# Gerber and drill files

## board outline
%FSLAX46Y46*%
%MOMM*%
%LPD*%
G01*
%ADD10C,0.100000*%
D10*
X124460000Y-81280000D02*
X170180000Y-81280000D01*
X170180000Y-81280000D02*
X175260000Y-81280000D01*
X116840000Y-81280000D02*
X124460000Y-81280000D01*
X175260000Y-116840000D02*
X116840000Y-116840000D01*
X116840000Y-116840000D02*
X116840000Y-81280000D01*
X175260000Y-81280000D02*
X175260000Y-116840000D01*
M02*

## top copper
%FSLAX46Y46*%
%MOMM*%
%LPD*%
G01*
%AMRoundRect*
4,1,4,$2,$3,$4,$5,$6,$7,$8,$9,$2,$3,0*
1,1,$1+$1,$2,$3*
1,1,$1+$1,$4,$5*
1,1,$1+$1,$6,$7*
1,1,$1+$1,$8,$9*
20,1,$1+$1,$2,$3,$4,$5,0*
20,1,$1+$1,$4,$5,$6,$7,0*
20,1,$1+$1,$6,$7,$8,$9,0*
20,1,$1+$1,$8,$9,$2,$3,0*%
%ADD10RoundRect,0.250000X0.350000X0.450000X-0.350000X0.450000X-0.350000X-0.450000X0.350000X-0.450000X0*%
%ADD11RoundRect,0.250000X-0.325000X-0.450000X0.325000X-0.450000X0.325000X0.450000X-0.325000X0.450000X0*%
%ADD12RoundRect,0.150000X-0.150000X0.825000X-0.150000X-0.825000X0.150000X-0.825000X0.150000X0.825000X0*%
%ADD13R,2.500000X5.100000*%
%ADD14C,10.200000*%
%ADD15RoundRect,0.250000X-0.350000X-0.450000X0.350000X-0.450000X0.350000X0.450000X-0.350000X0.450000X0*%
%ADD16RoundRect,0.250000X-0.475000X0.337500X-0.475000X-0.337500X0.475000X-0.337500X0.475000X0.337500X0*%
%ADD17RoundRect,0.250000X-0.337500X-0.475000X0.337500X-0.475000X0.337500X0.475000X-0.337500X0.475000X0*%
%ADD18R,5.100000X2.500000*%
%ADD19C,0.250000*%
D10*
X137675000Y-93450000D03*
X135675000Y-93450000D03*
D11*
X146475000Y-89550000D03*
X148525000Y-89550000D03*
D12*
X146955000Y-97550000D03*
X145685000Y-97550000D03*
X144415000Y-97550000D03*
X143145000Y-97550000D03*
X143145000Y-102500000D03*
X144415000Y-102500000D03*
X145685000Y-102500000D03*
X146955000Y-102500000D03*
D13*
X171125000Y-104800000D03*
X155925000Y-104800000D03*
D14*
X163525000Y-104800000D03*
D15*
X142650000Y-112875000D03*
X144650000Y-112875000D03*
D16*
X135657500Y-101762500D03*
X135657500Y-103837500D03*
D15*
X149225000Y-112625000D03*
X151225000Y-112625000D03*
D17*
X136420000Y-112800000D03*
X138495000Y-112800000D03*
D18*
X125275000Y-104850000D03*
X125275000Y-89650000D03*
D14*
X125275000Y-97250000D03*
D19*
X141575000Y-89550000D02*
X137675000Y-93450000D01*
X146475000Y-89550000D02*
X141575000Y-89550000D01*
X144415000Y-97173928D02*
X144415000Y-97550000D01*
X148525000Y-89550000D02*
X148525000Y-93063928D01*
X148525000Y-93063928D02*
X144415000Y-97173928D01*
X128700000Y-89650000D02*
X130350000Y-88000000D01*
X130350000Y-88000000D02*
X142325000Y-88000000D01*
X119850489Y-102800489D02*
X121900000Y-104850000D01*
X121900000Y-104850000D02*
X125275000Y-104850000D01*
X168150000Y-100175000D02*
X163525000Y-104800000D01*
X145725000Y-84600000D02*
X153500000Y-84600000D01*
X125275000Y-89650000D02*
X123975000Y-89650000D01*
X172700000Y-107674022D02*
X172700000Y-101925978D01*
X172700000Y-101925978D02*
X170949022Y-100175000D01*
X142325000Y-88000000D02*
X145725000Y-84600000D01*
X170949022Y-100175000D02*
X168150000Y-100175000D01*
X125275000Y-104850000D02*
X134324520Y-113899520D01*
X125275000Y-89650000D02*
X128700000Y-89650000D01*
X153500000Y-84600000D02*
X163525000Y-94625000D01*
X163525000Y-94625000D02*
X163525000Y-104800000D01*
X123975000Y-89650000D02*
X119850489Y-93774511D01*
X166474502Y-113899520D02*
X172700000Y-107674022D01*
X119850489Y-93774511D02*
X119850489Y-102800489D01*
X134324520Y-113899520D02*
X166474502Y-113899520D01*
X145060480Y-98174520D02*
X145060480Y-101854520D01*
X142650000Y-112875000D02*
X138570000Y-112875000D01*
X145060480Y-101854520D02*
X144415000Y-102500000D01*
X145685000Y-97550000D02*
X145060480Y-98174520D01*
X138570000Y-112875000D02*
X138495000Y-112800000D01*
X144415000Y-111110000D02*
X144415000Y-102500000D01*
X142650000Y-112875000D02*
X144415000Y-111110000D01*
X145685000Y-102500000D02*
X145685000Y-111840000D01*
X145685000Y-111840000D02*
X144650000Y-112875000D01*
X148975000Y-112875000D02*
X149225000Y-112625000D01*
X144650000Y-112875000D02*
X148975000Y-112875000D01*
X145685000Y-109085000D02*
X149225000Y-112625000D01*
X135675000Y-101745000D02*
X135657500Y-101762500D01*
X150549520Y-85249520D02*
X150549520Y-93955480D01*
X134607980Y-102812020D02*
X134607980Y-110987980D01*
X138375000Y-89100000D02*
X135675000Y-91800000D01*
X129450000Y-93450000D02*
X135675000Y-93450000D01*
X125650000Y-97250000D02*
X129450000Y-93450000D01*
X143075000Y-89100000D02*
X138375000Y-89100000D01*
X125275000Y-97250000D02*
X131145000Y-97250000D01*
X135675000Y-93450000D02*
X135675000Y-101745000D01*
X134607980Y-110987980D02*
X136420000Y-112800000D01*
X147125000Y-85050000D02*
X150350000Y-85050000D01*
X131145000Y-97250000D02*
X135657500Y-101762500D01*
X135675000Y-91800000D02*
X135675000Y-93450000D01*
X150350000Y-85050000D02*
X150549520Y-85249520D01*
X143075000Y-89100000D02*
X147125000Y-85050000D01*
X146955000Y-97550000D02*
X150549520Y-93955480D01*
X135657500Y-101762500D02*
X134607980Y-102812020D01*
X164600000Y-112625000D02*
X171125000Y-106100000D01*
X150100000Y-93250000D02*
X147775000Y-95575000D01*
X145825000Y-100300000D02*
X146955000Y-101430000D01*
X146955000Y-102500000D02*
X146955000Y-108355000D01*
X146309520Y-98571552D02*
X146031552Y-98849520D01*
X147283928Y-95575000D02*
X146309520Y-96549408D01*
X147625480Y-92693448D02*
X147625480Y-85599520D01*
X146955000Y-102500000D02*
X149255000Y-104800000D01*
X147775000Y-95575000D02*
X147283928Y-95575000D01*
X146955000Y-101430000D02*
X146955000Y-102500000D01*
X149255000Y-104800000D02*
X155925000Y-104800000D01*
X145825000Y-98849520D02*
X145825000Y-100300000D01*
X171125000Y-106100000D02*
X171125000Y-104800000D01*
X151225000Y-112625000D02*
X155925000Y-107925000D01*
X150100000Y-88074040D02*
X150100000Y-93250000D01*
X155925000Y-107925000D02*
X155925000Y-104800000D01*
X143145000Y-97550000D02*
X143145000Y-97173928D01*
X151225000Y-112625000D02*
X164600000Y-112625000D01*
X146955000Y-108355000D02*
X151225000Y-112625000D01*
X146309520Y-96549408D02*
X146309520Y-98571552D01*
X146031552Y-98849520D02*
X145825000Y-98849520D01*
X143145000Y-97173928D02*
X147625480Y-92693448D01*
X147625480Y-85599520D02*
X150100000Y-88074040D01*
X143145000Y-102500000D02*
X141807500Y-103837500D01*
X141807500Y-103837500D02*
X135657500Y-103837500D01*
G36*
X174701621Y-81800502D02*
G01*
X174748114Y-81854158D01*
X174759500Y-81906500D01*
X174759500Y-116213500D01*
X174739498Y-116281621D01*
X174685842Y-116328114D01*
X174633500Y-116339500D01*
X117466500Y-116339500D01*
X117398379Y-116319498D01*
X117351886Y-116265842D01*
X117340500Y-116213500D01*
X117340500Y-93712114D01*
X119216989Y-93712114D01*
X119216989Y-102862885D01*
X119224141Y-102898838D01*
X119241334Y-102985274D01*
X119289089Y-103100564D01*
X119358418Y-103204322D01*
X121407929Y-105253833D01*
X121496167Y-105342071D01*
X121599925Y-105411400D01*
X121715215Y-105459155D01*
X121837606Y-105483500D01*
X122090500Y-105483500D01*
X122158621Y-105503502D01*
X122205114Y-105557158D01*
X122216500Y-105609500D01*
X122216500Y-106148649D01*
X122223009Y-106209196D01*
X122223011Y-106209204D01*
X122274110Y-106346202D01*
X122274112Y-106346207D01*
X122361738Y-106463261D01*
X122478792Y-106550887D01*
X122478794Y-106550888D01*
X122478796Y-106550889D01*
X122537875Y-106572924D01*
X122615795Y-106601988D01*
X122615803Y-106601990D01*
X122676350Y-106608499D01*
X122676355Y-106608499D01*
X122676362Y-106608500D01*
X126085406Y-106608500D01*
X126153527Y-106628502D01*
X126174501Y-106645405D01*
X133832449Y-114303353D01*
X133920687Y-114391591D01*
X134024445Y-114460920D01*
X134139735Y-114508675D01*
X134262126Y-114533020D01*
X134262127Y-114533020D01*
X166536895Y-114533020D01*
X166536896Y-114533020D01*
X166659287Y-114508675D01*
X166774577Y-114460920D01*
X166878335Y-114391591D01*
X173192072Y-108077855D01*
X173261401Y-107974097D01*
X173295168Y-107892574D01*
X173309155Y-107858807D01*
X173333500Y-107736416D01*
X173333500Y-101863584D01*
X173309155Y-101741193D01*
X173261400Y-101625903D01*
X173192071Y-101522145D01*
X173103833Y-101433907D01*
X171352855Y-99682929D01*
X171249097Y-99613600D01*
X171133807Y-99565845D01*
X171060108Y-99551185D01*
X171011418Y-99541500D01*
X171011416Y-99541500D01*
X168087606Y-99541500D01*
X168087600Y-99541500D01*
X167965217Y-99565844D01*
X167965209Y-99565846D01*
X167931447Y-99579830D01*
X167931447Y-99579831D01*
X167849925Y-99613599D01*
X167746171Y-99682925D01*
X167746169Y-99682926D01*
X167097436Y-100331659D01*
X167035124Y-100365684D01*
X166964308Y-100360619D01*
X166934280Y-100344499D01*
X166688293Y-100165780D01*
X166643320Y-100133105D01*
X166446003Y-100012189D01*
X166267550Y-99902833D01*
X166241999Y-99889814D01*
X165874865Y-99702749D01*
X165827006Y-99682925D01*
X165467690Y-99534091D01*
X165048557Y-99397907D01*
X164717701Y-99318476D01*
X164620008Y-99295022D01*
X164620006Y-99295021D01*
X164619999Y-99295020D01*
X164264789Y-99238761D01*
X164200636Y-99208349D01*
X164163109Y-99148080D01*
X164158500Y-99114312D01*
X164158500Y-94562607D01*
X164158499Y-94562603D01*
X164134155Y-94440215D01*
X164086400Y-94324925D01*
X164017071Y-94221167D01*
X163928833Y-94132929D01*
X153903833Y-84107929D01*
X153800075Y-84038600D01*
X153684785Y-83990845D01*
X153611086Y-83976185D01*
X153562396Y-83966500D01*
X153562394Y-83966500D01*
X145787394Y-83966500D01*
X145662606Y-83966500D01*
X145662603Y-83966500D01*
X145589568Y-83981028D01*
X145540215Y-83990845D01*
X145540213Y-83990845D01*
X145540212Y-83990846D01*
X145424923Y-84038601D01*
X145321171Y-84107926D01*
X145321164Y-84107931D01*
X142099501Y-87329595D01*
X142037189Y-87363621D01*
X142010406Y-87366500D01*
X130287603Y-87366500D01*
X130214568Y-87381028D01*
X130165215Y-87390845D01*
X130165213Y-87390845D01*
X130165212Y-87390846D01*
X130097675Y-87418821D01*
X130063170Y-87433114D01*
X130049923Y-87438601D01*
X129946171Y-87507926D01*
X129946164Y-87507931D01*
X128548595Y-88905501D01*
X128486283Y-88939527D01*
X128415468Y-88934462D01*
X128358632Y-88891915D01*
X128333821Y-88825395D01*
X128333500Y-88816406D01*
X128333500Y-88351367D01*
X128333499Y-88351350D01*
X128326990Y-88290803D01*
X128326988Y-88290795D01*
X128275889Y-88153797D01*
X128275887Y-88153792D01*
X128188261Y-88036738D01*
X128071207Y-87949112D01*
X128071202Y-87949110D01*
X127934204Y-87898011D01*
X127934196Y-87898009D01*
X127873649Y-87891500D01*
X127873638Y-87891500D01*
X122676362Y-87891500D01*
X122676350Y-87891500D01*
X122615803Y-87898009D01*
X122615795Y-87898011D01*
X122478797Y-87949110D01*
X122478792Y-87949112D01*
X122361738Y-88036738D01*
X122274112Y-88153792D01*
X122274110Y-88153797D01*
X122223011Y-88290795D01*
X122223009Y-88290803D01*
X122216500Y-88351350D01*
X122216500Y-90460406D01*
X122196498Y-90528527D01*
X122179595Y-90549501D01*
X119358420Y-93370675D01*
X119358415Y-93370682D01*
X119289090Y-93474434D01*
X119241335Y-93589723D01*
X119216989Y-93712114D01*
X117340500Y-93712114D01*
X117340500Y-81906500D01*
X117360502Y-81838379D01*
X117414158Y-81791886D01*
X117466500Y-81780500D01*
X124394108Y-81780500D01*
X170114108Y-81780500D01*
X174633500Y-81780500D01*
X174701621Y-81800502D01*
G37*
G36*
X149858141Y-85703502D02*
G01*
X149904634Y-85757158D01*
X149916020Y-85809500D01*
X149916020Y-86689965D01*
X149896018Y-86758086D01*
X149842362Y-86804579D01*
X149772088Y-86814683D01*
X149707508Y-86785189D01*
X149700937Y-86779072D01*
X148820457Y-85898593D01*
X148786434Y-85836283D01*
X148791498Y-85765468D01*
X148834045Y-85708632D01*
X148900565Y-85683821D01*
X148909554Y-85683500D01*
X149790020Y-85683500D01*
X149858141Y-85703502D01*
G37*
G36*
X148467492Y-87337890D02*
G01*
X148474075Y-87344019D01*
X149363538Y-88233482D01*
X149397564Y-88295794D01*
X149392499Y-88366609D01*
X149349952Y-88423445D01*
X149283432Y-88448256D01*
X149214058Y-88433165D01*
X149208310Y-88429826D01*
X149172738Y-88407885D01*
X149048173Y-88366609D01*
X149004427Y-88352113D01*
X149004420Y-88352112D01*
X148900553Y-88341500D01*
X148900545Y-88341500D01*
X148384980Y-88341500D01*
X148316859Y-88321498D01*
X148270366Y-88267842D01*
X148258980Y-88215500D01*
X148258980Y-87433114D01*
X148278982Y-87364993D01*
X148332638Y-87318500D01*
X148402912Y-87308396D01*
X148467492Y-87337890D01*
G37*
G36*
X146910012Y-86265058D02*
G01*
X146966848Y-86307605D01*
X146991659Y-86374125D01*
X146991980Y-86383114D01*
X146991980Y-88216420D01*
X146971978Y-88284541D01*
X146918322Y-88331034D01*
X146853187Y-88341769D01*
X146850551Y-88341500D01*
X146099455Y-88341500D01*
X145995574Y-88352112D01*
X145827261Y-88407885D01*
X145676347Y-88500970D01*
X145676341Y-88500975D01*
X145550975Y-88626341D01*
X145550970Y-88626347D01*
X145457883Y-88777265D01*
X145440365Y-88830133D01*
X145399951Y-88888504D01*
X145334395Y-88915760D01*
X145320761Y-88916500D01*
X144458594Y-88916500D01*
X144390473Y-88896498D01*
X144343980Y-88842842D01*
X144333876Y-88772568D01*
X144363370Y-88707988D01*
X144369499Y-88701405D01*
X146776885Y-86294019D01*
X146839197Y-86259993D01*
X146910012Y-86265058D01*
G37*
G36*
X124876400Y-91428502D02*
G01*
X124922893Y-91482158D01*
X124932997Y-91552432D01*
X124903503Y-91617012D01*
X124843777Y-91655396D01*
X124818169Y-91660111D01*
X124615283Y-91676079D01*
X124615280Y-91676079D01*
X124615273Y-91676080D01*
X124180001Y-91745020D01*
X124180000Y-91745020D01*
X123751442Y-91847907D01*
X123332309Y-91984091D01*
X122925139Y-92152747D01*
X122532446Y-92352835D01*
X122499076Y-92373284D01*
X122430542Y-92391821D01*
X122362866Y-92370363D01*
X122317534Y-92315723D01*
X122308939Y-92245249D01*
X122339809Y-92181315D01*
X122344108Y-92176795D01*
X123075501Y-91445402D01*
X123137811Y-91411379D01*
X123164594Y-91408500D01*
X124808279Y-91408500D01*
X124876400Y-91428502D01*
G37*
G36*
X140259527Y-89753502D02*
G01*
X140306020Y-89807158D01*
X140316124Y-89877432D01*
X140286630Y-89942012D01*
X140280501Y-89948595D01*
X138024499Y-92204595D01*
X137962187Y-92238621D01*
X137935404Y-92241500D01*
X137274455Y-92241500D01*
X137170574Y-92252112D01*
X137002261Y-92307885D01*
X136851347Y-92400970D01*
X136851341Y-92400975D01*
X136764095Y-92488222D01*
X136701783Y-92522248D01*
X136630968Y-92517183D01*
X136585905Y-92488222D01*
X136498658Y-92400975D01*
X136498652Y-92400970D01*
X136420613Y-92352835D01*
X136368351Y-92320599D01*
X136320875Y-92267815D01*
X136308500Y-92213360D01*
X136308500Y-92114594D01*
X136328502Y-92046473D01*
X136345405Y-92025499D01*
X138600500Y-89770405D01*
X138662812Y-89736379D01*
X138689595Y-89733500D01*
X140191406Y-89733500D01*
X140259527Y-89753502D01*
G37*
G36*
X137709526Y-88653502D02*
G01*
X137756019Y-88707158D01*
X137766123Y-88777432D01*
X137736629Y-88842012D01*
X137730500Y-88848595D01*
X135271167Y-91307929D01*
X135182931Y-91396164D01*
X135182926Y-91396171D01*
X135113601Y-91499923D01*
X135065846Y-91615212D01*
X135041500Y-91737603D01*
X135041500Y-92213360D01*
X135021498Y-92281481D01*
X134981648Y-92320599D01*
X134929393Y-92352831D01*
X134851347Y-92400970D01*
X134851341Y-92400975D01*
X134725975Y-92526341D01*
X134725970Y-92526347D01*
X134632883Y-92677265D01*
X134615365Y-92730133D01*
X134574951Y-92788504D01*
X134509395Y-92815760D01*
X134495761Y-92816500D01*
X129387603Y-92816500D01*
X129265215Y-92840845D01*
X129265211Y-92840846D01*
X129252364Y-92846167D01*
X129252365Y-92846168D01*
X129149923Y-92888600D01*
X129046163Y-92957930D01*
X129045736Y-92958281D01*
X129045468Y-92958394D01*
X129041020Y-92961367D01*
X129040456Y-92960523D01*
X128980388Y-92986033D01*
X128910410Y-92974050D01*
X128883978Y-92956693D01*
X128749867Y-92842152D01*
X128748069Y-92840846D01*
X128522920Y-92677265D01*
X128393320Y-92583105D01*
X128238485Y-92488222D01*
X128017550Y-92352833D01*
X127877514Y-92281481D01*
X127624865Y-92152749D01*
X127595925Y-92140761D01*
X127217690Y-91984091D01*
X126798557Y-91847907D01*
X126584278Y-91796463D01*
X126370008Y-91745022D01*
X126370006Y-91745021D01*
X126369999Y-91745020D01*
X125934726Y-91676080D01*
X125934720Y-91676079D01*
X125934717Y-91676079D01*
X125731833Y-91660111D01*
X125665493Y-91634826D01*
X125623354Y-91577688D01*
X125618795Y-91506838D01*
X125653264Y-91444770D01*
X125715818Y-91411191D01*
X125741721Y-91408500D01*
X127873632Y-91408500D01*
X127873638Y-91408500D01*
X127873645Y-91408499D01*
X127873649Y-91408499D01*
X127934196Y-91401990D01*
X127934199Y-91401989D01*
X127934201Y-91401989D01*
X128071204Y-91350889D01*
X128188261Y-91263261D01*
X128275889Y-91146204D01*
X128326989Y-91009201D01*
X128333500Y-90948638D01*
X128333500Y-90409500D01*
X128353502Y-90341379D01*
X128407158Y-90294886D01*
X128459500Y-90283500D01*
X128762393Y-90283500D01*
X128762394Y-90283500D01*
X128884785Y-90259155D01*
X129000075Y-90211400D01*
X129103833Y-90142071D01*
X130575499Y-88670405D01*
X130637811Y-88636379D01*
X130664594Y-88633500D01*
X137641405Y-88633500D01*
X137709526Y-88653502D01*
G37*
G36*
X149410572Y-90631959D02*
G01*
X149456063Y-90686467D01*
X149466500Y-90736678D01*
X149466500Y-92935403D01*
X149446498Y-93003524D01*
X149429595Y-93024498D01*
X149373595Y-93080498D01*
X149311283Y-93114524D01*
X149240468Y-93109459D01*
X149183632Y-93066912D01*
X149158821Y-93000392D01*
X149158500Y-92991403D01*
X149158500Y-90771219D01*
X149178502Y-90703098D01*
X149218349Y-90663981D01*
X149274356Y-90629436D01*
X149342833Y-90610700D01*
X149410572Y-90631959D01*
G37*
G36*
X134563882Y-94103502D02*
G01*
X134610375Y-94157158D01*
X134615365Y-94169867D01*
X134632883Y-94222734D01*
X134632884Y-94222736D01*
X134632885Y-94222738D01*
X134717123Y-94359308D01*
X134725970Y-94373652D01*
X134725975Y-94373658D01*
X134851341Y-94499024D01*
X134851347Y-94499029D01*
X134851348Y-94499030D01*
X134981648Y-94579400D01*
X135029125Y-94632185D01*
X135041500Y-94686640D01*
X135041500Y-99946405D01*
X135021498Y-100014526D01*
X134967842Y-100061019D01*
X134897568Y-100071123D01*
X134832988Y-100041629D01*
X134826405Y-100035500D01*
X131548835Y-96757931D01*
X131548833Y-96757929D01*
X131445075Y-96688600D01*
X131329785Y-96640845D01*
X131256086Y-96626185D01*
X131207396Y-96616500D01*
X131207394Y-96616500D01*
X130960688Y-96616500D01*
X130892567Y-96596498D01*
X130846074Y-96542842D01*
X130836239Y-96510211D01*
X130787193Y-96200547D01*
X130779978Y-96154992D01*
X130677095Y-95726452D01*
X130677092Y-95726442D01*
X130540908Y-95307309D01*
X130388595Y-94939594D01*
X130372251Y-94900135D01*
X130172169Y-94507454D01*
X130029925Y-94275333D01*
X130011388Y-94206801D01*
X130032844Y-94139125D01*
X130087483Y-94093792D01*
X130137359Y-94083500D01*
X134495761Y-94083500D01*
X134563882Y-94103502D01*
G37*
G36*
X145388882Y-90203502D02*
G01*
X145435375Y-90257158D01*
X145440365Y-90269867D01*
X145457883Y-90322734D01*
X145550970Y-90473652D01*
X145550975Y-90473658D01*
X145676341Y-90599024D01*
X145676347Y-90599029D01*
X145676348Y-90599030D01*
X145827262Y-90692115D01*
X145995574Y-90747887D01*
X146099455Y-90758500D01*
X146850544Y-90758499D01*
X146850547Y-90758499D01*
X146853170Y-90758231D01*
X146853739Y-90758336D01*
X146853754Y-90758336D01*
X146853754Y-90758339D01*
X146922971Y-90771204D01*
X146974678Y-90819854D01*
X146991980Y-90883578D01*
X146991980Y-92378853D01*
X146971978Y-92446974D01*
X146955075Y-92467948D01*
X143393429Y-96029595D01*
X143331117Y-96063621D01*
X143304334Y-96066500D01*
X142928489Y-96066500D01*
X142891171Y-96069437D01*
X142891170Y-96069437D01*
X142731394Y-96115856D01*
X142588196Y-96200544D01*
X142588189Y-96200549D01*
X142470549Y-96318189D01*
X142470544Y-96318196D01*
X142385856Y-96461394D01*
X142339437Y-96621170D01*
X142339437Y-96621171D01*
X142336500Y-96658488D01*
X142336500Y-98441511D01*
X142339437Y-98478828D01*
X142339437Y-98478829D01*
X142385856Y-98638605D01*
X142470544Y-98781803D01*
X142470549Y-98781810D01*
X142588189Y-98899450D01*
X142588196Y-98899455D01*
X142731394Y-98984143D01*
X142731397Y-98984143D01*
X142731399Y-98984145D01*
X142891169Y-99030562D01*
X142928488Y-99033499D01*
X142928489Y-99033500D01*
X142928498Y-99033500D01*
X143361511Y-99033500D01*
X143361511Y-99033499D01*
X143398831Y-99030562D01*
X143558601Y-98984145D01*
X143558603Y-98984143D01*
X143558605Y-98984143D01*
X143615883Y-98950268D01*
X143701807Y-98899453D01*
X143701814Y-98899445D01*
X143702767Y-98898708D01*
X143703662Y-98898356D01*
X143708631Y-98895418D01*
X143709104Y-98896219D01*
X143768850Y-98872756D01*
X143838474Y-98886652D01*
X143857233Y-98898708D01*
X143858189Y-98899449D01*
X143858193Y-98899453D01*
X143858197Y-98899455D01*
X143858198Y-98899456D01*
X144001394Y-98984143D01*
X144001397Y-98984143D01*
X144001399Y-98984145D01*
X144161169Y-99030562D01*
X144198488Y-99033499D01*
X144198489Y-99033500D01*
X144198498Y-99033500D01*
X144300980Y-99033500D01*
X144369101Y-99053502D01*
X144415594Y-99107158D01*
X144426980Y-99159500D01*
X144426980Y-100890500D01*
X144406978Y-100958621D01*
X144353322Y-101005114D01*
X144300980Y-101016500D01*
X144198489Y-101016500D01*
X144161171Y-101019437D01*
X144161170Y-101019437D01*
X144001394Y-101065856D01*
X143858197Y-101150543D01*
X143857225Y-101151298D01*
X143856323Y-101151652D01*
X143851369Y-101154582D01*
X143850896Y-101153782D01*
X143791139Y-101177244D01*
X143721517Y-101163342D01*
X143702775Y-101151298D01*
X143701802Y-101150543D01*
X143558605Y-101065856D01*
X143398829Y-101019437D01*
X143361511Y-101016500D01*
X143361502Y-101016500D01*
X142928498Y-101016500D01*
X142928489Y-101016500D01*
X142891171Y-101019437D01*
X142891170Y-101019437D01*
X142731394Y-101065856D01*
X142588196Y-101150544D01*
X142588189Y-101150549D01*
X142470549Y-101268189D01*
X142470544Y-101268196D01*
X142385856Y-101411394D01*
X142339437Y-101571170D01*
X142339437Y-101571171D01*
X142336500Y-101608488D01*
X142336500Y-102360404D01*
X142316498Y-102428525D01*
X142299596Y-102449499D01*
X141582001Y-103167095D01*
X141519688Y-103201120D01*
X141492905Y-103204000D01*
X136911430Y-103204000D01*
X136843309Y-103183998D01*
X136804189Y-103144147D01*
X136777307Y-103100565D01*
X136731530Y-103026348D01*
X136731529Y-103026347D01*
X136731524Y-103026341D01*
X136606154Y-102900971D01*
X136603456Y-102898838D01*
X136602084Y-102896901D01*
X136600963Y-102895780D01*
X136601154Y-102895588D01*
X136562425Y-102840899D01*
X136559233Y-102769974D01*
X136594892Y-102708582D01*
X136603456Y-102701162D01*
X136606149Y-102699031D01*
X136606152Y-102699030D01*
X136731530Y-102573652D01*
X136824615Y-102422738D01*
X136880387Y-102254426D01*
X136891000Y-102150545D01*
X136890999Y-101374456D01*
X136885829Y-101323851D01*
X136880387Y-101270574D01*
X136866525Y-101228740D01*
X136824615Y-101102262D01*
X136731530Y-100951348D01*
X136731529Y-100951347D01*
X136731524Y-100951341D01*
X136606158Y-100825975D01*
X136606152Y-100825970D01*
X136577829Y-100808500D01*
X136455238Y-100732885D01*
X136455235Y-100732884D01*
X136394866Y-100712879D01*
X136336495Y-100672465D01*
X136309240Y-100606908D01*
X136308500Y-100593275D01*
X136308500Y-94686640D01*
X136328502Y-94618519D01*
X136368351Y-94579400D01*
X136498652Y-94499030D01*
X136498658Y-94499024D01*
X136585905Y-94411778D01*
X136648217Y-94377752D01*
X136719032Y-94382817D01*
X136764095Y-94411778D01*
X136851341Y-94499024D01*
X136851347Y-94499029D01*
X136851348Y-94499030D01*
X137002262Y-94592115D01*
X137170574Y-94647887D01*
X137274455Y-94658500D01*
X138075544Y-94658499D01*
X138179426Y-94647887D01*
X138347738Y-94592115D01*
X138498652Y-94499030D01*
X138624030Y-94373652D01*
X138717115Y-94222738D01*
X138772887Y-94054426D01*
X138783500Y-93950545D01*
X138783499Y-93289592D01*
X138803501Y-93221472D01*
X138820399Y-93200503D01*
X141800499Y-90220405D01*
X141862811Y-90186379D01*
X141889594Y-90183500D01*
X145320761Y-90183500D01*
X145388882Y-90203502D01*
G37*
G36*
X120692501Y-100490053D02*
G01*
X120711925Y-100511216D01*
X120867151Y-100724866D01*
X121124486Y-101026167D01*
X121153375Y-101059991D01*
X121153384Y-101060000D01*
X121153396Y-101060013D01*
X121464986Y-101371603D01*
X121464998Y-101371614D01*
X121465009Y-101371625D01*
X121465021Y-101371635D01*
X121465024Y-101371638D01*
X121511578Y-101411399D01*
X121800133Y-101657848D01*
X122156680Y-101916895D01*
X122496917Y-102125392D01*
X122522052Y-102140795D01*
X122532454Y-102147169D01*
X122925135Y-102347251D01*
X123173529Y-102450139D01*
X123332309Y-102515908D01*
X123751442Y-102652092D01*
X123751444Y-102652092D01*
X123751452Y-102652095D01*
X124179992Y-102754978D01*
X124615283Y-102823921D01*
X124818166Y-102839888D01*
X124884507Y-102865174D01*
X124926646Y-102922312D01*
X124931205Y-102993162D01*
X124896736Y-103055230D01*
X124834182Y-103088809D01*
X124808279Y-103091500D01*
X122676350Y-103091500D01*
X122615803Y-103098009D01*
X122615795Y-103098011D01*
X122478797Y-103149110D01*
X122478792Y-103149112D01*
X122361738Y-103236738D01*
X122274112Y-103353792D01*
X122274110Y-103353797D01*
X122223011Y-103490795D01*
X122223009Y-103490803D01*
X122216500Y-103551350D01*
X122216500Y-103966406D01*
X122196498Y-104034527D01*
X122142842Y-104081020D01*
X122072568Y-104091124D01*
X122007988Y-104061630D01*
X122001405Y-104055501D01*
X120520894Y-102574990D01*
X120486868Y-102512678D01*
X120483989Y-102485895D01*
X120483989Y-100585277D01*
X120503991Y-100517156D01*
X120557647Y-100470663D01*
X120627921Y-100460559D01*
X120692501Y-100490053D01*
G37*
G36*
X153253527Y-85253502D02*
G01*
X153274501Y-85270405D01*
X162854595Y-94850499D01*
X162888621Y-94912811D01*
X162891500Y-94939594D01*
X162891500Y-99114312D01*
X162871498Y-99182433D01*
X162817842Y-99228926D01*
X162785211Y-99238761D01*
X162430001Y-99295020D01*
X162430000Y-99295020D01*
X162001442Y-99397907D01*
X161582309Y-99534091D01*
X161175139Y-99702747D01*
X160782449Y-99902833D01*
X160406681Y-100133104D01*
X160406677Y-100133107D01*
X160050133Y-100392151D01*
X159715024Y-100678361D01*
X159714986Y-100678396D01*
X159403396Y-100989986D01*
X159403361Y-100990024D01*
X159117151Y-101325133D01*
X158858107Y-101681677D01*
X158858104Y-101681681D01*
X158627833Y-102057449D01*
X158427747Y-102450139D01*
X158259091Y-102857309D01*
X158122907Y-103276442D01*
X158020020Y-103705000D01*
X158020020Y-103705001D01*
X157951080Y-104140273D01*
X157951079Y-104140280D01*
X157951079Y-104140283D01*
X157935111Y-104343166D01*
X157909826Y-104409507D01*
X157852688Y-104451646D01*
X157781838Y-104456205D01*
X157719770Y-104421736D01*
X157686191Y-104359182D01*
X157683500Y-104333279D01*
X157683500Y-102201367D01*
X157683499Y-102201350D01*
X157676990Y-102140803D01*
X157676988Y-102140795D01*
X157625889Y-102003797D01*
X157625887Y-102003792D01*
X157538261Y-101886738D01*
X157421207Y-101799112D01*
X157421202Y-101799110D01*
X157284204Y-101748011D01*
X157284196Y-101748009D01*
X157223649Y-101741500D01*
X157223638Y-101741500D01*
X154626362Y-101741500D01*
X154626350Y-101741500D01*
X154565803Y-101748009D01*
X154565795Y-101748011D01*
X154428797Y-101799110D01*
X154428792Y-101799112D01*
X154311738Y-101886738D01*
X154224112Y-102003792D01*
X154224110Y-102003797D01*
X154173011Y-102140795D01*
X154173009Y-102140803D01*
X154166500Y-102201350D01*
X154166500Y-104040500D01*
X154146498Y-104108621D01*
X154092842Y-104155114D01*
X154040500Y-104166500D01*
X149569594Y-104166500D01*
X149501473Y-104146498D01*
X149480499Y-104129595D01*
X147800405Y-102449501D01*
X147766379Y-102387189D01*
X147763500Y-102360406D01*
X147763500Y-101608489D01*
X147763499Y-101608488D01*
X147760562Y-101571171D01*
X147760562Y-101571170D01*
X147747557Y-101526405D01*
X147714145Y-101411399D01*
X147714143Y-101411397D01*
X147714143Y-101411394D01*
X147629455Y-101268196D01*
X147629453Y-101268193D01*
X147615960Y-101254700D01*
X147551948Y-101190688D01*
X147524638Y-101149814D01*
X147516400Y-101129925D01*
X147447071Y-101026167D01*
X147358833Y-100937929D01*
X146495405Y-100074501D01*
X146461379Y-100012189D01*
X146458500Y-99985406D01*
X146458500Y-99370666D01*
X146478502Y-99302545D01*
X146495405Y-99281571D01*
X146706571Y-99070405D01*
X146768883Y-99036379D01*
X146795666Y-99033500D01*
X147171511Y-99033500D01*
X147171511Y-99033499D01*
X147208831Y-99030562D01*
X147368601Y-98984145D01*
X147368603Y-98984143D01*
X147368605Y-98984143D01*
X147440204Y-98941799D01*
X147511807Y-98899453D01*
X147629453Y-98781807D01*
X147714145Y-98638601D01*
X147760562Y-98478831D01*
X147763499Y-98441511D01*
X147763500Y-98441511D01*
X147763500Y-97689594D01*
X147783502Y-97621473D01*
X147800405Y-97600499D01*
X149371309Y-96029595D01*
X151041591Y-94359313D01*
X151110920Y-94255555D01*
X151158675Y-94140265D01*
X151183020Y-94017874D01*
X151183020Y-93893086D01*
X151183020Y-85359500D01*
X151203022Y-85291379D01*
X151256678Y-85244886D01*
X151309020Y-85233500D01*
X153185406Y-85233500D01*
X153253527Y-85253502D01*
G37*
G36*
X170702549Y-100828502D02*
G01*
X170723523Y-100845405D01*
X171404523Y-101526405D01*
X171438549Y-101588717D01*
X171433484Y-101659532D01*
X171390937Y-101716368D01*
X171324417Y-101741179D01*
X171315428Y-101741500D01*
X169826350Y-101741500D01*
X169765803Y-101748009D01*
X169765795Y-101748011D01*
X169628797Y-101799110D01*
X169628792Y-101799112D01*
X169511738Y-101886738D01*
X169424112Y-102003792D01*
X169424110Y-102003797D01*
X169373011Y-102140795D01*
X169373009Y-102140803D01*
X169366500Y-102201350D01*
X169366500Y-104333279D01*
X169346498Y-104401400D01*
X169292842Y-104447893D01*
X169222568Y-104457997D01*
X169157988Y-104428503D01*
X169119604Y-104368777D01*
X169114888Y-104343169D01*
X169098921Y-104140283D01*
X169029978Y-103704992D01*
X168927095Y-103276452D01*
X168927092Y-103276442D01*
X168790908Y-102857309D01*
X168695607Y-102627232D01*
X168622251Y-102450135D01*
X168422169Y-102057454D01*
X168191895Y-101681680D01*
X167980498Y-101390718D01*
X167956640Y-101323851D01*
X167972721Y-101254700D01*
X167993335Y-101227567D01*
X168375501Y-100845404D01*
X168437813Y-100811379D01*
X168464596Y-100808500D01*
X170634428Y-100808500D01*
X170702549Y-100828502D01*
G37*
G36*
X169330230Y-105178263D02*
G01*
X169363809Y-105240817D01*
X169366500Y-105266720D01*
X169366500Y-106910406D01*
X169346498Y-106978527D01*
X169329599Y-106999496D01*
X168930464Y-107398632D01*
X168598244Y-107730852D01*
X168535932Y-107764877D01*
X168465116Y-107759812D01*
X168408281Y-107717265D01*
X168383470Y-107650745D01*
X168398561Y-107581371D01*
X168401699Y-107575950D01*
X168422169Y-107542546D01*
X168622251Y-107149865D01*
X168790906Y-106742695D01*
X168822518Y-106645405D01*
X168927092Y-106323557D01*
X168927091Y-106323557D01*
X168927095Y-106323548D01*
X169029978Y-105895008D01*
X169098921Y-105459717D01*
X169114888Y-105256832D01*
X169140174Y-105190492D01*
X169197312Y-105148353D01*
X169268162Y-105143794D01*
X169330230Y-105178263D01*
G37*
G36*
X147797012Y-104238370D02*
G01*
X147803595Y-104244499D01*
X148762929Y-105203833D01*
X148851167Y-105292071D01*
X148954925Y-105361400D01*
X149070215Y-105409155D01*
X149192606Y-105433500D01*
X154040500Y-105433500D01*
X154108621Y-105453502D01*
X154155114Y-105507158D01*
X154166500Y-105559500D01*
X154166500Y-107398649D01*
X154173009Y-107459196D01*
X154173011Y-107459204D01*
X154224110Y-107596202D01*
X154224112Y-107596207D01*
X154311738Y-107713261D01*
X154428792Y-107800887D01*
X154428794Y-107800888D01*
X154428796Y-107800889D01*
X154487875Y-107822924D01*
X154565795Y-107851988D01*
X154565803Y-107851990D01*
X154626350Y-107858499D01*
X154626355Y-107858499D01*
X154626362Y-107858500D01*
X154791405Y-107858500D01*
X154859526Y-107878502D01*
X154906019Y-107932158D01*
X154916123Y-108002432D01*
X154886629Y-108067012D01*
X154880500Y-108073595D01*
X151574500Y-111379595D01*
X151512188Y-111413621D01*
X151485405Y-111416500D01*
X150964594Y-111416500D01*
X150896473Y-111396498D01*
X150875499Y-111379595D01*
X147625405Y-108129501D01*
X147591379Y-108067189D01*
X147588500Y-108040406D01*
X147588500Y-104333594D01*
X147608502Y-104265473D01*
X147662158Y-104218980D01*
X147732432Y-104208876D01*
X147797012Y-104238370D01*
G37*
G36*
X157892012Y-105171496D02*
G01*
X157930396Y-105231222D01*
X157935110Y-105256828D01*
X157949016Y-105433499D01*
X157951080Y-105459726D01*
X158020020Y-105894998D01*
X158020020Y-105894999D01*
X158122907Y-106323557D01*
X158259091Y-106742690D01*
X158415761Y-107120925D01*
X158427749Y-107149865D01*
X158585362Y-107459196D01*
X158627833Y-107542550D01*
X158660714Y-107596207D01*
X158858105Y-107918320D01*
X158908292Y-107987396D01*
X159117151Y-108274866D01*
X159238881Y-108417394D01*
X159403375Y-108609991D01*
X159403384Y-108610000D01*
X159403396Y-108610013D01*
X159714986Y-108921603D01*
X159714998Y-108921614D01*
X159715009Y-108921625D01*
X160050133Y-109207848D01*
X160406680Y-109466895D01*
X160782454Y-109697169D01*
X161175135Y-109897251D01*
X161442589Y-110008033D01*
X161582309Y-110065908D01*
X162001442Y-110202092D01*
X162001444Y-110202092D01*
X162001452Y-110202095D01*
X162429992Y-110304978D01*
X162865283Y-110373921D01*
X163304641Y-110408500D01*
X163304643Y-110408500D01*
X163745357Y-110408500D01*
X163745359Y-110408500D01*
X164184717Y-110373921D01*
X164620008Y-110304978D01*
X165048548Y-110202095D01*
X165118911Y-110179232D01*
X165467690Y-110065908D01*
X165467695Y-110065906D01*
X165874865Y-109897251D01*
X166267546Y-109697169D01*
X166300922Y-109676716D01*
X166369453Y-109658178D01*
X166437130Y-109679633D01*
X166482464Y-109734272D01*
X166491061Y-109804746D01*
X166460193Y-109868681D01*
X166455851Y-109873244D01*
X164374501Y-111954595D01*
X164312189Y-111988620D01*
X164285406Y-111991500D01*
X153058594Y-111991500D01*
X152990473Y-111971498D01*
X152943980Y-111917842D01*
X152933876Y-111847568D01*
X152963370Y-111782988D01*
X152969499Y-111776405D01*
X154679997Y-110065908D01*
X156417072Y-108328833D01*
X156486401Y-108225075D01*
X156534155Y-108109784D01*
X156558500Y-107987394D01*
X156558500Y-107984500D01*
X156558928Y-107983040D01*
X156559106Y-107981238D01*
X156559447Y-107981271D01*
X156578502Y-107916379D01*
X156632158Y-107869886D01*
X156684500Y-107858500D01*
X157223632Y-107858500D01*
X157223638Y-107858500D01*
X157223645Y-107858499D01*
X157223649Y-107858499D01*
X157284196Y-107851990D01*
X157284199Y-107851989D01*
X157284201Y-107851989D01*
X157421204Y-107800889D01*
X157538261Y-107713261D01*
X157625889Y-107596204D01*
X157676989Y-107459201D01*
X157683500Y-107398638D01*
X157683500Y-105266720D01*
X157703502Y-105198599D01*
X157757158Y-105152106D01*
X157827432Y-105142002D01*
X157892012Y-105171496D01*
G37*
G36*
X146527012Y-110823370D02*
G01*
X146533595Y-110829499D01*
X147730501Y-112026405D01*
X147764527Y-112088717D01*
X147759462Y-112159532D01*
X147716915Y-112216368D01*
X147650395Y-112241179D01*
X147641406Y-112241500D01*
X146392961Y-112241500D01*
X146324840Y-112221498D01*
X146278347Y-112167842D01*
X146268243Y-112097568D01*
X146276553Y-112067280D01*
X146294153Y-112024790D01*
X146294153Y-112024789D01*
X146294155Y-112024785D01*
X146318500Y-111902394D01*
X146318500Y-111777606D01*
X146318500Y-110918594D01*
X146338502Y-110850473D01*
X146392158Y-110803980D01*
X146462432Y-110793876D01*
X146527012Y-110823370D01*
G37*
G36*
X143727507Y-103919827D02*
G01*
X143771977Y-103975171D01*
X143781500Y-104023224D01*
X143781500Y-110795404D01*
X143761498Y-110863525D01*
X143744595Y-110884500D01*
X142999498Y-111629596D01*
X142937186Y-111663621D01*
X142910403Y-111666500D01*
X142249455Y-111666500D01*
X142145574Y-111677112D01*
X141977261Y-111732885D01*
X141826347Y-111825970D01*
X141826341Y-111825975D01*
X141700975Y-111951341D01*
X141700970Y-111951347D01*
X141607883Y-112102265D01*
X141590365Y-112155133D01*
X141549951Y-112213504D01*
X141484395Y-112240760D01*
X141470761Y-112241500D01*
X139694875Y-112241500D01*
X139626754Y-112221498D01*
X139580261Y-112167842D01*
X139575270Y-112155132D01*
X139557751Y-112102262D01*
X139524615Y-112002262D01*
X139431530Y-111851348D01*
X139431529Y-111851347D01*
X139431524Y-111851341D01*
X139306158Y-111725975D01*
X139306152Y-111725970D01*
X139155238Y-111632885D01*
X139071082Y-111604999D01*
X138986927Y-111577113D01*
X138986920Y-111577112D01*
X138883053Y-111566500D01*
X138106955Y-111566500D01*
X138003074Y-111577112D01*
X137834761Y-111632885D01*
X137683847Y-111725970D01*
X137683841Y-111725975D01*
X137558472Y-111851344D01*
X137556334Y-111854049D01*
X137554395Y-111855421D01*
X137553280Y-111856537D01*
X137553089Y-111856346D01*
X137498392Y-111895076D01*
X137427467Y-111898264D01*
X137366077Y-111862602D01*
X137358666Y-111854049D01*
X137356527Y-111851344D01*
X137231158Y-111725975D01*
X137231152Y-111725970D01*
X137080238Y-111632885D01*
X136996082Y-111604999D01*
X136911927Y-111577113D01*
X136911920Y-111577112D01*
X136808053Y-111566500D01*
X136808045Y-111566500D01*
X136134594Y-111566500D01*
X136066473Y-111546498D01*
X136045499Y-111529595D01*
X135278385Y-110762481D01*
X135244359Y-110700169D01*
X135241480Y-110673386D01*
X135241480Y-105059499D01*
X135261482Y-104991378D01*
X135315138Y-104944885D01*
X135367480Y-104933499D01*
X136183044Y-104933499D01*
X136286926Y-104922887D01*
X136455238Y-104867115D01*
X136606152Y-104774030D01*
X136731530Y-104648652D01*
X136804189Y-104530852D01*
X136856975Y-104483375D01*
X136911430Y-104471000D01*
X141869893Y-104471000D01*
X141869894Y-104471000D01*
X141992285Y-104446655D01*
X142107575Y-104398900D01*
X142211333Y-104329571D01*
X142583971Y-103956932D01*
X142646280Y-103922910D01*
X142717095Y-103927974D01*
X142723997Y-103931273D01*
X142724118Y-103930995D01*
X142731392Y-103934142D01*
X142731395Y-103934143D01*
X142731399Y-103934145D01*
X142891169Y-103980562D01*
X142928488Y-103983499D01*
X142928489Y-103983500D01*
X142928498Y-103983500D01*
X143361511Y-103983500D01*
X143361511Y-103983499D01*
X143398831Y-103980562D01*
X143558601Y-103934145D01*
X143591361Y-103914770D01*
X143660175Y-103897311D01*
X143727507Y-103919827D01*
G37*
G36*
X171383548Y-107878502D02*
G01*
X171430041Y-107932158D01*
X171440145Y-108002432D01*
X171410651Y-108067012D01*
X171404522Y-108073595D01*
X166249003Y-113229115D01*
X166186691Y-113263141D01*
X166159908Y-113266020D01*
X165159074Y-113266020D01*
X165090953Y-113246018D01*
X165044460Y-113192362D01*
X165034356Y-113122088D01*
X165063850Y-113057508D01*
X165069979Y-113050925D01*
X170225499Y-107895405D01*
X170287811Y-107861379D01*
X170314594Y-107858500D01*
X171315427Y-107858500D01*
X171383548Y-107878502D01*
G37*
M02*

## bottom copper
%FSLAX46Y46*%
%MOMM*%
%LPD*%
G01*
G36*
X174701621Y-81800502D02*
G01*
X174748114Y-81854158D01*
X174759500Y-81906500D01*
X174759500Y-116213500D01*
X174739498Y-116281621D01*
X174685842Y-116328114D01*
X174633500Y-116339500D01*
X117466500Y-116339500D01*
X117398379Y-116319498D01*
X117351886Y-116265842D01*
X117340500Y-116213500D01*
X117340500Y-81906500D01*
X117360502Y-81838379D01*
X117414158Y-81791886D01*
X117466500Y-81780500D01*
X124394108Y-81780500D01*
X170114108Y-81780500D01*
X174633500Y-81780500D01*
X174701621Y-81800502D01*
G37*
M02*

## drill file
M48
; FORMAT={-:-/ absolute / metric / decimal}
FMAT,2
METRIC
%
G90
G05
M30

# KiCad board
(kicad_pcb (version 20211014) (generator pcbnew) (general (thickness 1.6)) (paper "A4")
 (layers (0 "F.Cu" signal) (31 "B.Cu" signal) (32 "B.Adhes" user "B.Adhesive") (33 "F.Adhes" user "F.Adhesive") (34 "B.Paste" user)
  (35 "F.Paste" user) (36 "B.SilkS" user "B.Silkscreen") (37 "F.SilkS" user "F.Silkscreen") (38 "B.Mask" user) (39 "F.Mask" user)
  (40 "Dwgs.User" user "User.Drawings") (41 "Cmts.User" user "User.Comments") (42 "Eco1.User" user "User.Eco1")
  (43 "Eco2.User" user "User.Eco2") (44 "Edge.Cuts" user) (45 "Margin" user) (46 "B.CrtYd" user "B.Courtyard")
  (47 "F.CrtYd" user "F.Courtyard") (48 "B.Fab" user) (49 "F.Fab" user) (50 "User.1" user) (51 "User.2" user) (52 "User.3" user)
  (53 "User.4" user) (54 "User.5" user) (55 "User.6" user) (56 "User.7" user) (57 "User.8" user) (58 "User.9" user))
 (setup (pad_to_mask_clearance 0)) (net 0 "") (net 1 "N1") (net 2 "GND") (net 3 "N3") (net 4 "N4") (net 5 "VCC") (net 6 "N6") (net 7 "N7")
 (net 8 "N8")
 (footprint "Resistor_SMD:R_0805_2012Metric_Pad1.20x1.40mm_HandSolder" (layer "F.Cu") (at 136.675 93.45 180)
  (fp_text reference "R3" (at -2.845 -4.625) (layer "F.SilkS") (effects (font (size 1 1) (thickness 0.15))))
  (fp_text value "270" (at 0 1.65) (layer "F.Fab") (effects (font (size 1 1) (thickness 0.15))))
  (pad "1" smd roundrect (at -1 0 180) (size 1.2 1.4) (layers "F.Cu" "F.Paste" "F.Mask") (roundrect_rratio 0.2083333333) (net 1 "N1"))
  (pad "2" smd roundrect (at 1 0 180) (size 1.2 1.4) (layers "F.Cu" "F.Paste" "F.Mask") (roundrect_rratio 0.2083333333) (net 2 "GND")))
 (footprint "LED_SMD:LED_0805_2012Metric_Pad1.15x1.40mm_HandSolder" (layer "F.Cu") (at 147.5 89.55)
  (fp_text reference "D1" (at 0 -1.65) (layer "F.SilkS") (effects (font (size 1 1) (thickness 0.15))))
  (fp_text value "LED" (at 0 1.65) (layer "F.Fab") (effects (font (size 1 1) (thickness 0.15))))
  (pad "1" smd roundrect (at -1.025 0) (size 1.15 1.4) (layers "F.Cu" "F.Paste" "F.Mask") (roundrect_rratio 0.2173913043) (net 1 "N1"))
  (pad "2" smd roundrect (at 1.025 0) (size 1.15 1.4) (layers "F.Cu" "F.Paste" "F.Mask") (roundrect_rratio 0.2173913043) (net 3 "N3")))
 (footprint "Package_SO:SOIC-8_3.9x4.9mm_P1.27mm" (layer "F.Cu") (at 145.05 100.025 -90)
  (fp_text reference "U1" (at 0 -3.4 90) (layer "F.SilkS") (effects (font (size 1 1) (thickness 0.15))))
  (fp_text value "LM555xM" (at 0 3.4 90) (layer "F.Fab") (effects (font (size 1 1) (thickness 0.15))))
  (pad "1" smd roundrect (at -2.475 -1.905 270) (size 1.95 0.6) (layers "F.Cu" "F.Paste" "F.Mask") (roundrect_rratio 0.25) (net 2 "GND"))
  (pad "2" smd roundrect (at -2.475 -0.635 270) (size 1.95 0.6) (layers "F.Cu" "F.Paste" "F.Mask") (roundrect_rratio 0.25) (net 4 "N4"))
  (pad "3" smd roundrect (at -2.475 0.635 270) (size 1.95 0.6) (layers "F.Cu" "F.Paste" "F.Mask") (roundrect_rratio 0.25) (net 3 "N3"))
  (pad "4" smd roundrect (at -2.475 1.905 270) (size 1.95 0.6) (layers "F.Cu" "F.Paste" "F.Mask") (roundrect_rratio 0.25) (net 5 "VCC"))
  (pad "5" smd roundrect (at 2.475 1.905 270) (size 1.95 0.6) (layers "F.Cu" "F.Paste" "F.Mask") (roundrect_rratio 0.25) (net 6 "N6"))
  (pad "6" smd roundrect (at 2.475 0.635 270) (size 1.95 0.6) (layers "F.Cu" "F.Paste" "F.Mask") (roundrect_rratio 0.25) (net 4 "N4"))
  (pad "7" smd roundrect (at 2.475 -0.635 270) (size 1.95 0.6) (layers "F.Cu" "F.Paste" "F.Mask") (roundrect_rratio 0.25) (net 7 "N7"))
  (pad "8" smd roundrect (at 2.475 -1.905 270) (size 1.95 0.6) (layers "F.Cu" "F.Paste" "F.Mask") (roundrect_rratio 0.25) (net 5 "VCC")))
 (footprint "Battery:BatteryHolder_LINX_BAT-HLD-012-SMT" (layer "F.Cu") (at 163.525 104.8 180)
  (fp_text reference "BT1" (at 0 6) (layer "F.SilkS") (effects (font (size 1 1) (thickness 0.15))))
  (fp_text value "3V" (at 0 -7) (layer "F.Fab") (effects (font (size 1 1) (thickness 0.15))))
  (pad "1" smd rect (at -7.6 0 180) (size 2.5 5.1) (layers "F.Cu" "F.Paste" "F.Mask") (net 5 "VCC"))
  (pad "1" smd rect (at 7.6 0 180) (size 2.5 5.1) (layers "F.Cu" "F.Paste" "F.Mask") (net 5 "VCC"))
  (pad "2" smd circle (at 0 0 180) (size 10.2 10.2) (layers "F.Cu" "F.Mask") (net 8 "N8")))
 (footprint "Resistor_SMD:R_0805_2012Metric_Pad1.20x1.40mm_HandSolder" (layer "F.Cu") (at 143.65 112.875)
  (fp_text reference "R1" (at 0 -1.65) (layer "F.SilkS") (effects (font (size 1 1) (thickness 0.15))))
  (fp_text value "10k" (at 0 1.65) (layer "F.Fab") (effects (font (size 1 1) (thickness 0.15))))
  (pad "1" smd roundrect (at -1 0) (size 1.2 1.4) (layers "F.Cu" "F.Paste" "F.Mask") (roundrect_rratio 0.2083333333) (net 4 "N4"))
  (pad "2" smd roundrect (at 1 0) (size 1.2 1.4) (layers "F.Cu" "F.Paste" "F.Mask") (roundrect_rratio 0.2083333333) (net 7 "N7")))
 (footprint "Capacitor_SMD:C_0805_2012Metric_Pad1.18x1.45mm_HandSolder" (layer "F.Cu") (at 135.6575 102.8 -90)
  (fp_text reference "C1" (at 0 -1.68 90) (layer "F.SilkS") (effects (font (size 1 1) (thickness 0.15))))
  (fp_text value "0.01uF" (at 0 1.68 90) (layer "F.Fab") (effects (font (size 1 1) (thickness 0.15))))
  (pad "1" smd roundrect (at -1.0375 0 270) (size 1.175 1.45) (layers "F.Cu" "F.Paste" "F.Mask") (roundrect_rratio 0.2127659574)
   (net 2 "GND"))
  (pad "2" smd roundrect (at 1.0375 0 270) (size 1.175 1.45) (layers "F.Cu" "F.Paste" "F.Mask") (roundrect_rratio 0.2127659574) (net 6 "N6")))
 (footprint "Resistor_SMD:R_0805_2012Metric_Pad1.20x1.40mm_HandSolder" (layer "F.Cu") (at 150.225 112.625)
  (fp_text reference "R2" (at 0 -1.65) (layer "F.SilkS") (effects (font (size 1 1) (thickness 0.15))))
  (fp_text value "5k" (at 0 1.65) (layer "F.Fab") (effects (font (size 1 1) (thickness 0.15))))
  (pad "1" smd roundrect (at -1 0) (size 1.2 1.4) (layers "F.Cu" "F.Paste" "F.Mask") (roundrect_rratio 0.2083333333) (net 7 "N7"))
  (pad "2" smd roundrect (at 1 0) (size 1.2 1.4) (layers "F.Cu" "F.Paste" "F.Mask") (roundrect_rratio 0.2083333333) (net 5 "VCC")))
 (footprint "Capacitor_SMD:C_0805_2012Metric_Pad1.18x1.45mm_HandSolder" (layer "F.Cu") (at 137.4575 112.8)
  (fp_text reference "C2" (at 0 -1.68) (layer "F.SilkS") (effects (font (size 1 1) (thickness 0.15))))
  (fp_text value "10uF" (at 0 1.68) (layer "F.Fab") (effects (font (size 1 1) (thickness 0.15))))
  (pad "1" smd roundrect (at -1.0375 0) (size 1.175 1.45) (layers "F.Cu" "F.Paste" "F.Mask") (roundrect_rratio 0.2127659574) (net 2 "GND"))
  (pad "2" smd roundrect (at 1.0375 0) (size 1.175 1.45) (layers "F.Cu" "F.Paste" "F.Mask") (roundrect_rratio 0.2127659574) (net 4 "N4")))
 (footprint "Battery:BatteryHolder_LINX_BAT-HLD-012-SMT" (layer "F.Cu") (at 125.275 97.25 -90)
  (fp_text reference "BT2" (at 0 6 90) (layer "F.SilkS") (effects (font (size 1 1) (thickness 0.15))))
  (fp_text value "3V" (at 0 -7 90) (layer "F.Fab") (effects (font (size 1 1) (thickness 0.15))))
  (pad "1" smd rect (at 7.6 0 270) (size 2.5 5.1) (layers "F.Cu" "F.Paste" "F.Mask") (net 8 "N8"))
  (pad "1" smd rect (at -7.6 0 270) (size 2.5 5.1) (layers "F.Cu" "F.Paste" "F.Mask") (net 8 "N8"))
  (pad "2" smd circle (at 0 0 270) (size 10.2 10.2) (layers "F.Cu" "F.Mask") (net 2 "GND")))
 (gr_line (start 124.46 81.28) (end 170.18 81.28) (layer "Edge.Cuts") (width 0.1))
 (gr_line (start 170.18 81.28) (end 175.26 81.28) (layer "Edge.Cuts") (width 0.1))
 (gr_line (start 116.84 81.28) (end 124.46 81.28) (layer "Edge.Cuts") (width 0.1))
 (gr_line (start 175.26 116.84) (end 116.84 116.84) (layer "Edge.Cuts") (width 0.1))
 (gr_line (start 116.84 116.84) (end 116.84 81.28) (layer "Edge.Cuts") (width 0.1))
 (gr_line (start 175.26 81.28) (end 175.26 116.84) (layer "Edge.Cuts") (width 0.1))
 (segment (start 141.575 89.55) (end 137.675 93.45) (width 0.25) (layer "F.Cu") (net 1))
 (segment (start 146.475 89.55) (end 141.575 89.55) (width 0.25) (layer "F.Cu") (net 1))
 (segment (start 144.415 97.173928) (end 144.415 97.55) (width 0.25) (layer "F.Cu") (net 3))
 (segment (start 148.525 89.55) (end 148.525 93.063928) (width 0.25) (layer "F.Cu") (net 3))
 (segment (start 148.525 93.063928) (end 144.415 97.173928) (width 0.25) (layer "F.Cu") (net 3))
 (segment (start 128.7 89.65) (end 130.35 88) (width 0.25) (layer "F.Cu") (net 8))
 (segment (start 130.35 88) (end 142.325 88) (width 0.25) (layer "F.Cu") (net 8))
 (segment (start 119.850489 102.800489) (end 121.9 104.85) (width 0.25) (layer "F.Cu") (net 8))
 (segment (start 121.9 104.85) (end 125.275 104.85) (width 0.25) (layer "F.Cu") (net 8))
 (segment (start 168.15 100.175) (end 163.525 104.8) (width 0.25) (layer "F.Cu") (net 8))
 (segment (start 145.725 84.6) (end 153.5 84.6) (width 0.25) (layer "F.Cu") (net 8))
 (segment (start 125.275 89.65) (end 123.975 89.65) (width 0.25) (layer "F.Cu") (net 8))
 (segment (start 172.7 107.674022) (end 172.7 101.925978) (width 0.25) (layer "F.Cu") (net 8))
 (segment (start 172.7 101.925978) (end 170.949022 100.175) (width 0.25) (layer "F.Cu") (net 8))
 (segment (start 142.325 88) (end 145.725 84.6) (width 0.25) (layer "F.Cu") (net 8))
 (segment (start 170.949022 100.175) (end 168.15 100.175) (width 0.25) (layer "F.Cu") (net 8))
 (segment (start 125.275 104.85) (end 134.32452 113.89952) (width 0.25) (layer "F.Cu") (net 8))
 (segment (start 125.275 89.65) (end 128.7 89.65) (width 0.25) (layer "F.Cu") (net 8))
 (segment (start 153.5 84.6) (end 163.525 94.625) (width 0.25) (layer "F.Cu") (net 8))
 (segment (start 163.525 94.625) (end 163.525 104.8) (width 0.25) (layer "F.Cu") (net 8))
 (segment (start 123.975 89.65) (end 119.850489 93.774511) (width 0.25) (layer "F.Cu") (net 8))
 (segment (start 166.474502 113.89952) (end 172.7 107.674022) (width 0.25) (layer "F.Cu") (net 8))
 (segment (start 119.850489 93.774511) (end 119.850489 102.800489) (width 0.25) (layer "F.Cu") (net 8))
 (segment (start 134.32452 113.89952) (end 166.474502 113.89952) (width 0.25) (layer "F.Cu") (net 8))
 (segment (start 145.06048 98.17452) (end 145.06048 101.85452) (width 0.25) (layer "F.Cu") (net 4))
 (segment (start 142.65 112.875) (end 138.57 112.875) (width 0.25) (layer "F.Cu") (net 4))
 (segment (start 145.06048 101.85452) (end 144.415 102.5) (width 0.25) (layer "F.Cu") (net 4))
 (segment (start 145.685 97.55) (end 145.06048 98.17452) (width 0.25) (layer "F.Cu") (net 4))
 (segment (start 138.57 112.875) (end 138.495 112.8) (width 0.25) (layer "F.Cu") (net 4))
 (segment (start 144.415 111.11) (end 144.415 102.5) (width 0.25) (layer "F.Cu") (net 4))
 (segment (start 142.65 112.875) (end 144.415 111.11) (width 0.25) (layer "F.Cu") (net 4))
 (segment (start 145.685 102.5) (end 145.685 111.84) (width 0.25) (layer "F.Cu") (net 7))
 (segment (start 145.685 111.84) (end 144.65 112.875) (width 0.25) (layer "F.Cu") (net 7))
 (segment (start 148.975 112.875) (end 149.225 112.625) (width 0.25) (layer "F.Cu") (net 7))
 (segment (start 144.65 112.875) (end 148.975 112.875) (width 0.25) (layer "F.Cu") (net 7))
 (segment (start 145.685 109.085) (end 149.225 112.625) (width 0.25) (layer "F.Cu") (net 7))
 (segment (start 135.675 101.745) (end 135.6575 101.7625) (width 0.25) (layer "F.Cu") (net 2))
 (segment (start 150.54952 85.24952) (end 150.54952 93.95548) (width 0.25) (layer "F.Cu") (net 2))
 (segment (start 134.60798 102.81202) (end 134.60798 110.98798) (width 0.25) (layer "F.Cu") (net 2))
 (segment (start 138.375 89.1) (end 135.675 91.8) (width 0.25) (layer "F.Cu") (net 2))
 (segment (start 129.45 93.45) (end 135.675 93.45) (width 0.25) (layer "F.Cu") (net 2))
 (segment (start 125.65 97.25) (end 129.45 93.45) (width 0.25) (layer "F.Cu") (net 2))
 (segment (start 143.075 89.1) (end 138.375 89.1) (width 0.25) (layer "F.Cu") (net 2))
 (segment (start 125.275 97.25) (end 131.145 97.25) (width 0.25) (layer "F.Cu") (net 2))
 (segment (start 135.675 93.45) (end 135.675 101.745) (width 0.25) (layer "F.Cu") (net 2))
 (segment (start 134.60798 110.98798) (end 136.42 112.8) (width 0.25) (layer "F.Cu") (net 2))
 (segment (start 147.125 85.05) (end 150.35 85.05) (width 0.25) (layer "F.Cu") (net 2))
 (segment (start 131.145 97.25) (end 135.6575 101.7625) (width 0.25) (layer "F.Cu") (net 2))
 (segment (start 135.675 91.8) (end 135.675 93.45) (width 0.25) (layer "F.Cu") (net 2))
 (segment (start 150.35 85.05) (end 150.54952 85.24952) (width 0.25) (layer "F.Cu") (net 2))
 (segment (start 143.075 89.1) (end 147.125 85.05) (width 0.25) (layer "F.Cu") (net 2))
 (segment (start 146.955 97.55) (end 150.54952 93.95548) (width 0.25) (layer "F.Cu") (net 2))
 (segment (start 135.6575 101.7625) (end 134.60798 102.81202) (width 0.25) (layer "F.Cu") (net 2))
 (segment (start 164.6 112.625) (end 171.125 106.1) (width 0.25) (layer "F.Cu") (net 5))
 (segment (start 150.1 93.25) (end 147.775 95.575) (width 0.25) (layer "F.Cu") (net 5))
 (segment (start 145.825 100.3) (end 146.955 101.43) (width 0.25) (layer "F.Cu") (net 5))
 (segment (start 146.955 102.5) (end 146.955 108.355) (width 0.25) (layer "F.Cu") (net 5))
 (segment (start 146.30952 98.571552) (end 146.031552 98.84952) (width 0.25) (layer "F.Cu") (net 5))
 (segment (start 147.283928 95.575) (end 146.30952 96.549408) (width 0.25) (layer "F.Cu") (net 5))
 (segment (start 147.62548 92.693448) (end 147.62548 85.59952) (width 0.25) (layer "F.Cu") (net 5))
 (segment (start 146.955 102.5) (end 149.255 104.8) (width 0.25) (layer "F.Cu") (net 5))
 (segment (start 147.775 95.575) (end 147.283928 95.575) (width 0.25) (layer "F.Cu") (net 5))
 (segment (start 146.955 101.43) (end 146.955 102.5) (width 0.25) (layer "F.Cu") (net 5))
 (segment (start 149.255 104.8) (end 155.925 104.8) (width 0.25) (layer "F.Cu") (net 5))
 (segment (start 145.825 98.84952) (end 145.825 100.3) (width 0.25) (layer "F.Cu") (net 5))
 (segment (start 171.125 106.1) (end 171.125 104.8) (width 0.25) (layer "F.Cu") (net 5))
 (segment (start 151.225 112.625) (end 155.925 107.925) (width 0.25) (layer "F.Cu") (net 5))
 (segment (start 150.1 88.07404) (end 150.1 93.25) (width 0.25) (layer "F.Cu") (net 5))
 (segment (start 155.925 107.925) (end 155.925 104.8) (width 0.25) (layer "F.Cu") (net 5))
 (segment (start 143.145 97.55) (end 143.145 97.173928) (width 0.25) (layer "F.Cu") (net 5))
 (segment (start 151.225 112.625) (end 164.6 112.625) (width 0.25) (layer "F.Cu") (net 5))
 (segment (start 146.955 108.355) (end 151.225 112.625) (width 0.25) (layer "F.Cu") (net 5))
 (segment (start 146.30952 96.549408) (end 146.30952 98.571552) (width 0.25) (layer "F.Cu") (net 5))
 (segment (start 146.031552 98.84952) (end 145.825 98.84952) (width 0.25) (layer "F.Cu") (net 5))
 (segment (start 143.145 97.173928) (end 147.62548 92.693448) (width 0.25) (layer "F.Cu") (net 5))
 (segment (start 147.62548 85.59952) (end 150.1 88.07404) (width 0.25) (layer "F.Cu") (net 5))
 (segment (start 143.145 102.5) (end 141.8075 103.8375) (width 0.25) (layer "F.Cu") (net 6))
 (segment (start 141.8075 103.8375) (end 135.6575 103.8375) (width 0.25) (layer "F.Cu") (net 6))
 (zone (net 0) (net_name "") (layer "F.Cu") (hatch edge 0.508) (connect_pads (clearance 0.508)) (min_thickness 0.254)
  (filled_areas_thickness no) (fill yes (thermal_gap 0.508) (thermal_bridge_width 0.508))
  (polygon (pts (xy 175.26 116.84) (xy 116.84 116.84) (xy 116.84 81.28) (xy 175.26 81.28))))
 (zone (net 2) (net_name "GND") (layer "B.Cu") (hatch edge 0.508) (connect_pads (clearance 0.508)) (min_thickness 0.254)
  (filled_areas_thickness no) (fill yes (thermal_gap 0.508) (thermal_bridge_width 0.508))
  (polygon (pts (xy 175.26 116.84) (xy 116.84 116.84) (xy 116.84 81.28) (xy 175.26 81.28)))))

